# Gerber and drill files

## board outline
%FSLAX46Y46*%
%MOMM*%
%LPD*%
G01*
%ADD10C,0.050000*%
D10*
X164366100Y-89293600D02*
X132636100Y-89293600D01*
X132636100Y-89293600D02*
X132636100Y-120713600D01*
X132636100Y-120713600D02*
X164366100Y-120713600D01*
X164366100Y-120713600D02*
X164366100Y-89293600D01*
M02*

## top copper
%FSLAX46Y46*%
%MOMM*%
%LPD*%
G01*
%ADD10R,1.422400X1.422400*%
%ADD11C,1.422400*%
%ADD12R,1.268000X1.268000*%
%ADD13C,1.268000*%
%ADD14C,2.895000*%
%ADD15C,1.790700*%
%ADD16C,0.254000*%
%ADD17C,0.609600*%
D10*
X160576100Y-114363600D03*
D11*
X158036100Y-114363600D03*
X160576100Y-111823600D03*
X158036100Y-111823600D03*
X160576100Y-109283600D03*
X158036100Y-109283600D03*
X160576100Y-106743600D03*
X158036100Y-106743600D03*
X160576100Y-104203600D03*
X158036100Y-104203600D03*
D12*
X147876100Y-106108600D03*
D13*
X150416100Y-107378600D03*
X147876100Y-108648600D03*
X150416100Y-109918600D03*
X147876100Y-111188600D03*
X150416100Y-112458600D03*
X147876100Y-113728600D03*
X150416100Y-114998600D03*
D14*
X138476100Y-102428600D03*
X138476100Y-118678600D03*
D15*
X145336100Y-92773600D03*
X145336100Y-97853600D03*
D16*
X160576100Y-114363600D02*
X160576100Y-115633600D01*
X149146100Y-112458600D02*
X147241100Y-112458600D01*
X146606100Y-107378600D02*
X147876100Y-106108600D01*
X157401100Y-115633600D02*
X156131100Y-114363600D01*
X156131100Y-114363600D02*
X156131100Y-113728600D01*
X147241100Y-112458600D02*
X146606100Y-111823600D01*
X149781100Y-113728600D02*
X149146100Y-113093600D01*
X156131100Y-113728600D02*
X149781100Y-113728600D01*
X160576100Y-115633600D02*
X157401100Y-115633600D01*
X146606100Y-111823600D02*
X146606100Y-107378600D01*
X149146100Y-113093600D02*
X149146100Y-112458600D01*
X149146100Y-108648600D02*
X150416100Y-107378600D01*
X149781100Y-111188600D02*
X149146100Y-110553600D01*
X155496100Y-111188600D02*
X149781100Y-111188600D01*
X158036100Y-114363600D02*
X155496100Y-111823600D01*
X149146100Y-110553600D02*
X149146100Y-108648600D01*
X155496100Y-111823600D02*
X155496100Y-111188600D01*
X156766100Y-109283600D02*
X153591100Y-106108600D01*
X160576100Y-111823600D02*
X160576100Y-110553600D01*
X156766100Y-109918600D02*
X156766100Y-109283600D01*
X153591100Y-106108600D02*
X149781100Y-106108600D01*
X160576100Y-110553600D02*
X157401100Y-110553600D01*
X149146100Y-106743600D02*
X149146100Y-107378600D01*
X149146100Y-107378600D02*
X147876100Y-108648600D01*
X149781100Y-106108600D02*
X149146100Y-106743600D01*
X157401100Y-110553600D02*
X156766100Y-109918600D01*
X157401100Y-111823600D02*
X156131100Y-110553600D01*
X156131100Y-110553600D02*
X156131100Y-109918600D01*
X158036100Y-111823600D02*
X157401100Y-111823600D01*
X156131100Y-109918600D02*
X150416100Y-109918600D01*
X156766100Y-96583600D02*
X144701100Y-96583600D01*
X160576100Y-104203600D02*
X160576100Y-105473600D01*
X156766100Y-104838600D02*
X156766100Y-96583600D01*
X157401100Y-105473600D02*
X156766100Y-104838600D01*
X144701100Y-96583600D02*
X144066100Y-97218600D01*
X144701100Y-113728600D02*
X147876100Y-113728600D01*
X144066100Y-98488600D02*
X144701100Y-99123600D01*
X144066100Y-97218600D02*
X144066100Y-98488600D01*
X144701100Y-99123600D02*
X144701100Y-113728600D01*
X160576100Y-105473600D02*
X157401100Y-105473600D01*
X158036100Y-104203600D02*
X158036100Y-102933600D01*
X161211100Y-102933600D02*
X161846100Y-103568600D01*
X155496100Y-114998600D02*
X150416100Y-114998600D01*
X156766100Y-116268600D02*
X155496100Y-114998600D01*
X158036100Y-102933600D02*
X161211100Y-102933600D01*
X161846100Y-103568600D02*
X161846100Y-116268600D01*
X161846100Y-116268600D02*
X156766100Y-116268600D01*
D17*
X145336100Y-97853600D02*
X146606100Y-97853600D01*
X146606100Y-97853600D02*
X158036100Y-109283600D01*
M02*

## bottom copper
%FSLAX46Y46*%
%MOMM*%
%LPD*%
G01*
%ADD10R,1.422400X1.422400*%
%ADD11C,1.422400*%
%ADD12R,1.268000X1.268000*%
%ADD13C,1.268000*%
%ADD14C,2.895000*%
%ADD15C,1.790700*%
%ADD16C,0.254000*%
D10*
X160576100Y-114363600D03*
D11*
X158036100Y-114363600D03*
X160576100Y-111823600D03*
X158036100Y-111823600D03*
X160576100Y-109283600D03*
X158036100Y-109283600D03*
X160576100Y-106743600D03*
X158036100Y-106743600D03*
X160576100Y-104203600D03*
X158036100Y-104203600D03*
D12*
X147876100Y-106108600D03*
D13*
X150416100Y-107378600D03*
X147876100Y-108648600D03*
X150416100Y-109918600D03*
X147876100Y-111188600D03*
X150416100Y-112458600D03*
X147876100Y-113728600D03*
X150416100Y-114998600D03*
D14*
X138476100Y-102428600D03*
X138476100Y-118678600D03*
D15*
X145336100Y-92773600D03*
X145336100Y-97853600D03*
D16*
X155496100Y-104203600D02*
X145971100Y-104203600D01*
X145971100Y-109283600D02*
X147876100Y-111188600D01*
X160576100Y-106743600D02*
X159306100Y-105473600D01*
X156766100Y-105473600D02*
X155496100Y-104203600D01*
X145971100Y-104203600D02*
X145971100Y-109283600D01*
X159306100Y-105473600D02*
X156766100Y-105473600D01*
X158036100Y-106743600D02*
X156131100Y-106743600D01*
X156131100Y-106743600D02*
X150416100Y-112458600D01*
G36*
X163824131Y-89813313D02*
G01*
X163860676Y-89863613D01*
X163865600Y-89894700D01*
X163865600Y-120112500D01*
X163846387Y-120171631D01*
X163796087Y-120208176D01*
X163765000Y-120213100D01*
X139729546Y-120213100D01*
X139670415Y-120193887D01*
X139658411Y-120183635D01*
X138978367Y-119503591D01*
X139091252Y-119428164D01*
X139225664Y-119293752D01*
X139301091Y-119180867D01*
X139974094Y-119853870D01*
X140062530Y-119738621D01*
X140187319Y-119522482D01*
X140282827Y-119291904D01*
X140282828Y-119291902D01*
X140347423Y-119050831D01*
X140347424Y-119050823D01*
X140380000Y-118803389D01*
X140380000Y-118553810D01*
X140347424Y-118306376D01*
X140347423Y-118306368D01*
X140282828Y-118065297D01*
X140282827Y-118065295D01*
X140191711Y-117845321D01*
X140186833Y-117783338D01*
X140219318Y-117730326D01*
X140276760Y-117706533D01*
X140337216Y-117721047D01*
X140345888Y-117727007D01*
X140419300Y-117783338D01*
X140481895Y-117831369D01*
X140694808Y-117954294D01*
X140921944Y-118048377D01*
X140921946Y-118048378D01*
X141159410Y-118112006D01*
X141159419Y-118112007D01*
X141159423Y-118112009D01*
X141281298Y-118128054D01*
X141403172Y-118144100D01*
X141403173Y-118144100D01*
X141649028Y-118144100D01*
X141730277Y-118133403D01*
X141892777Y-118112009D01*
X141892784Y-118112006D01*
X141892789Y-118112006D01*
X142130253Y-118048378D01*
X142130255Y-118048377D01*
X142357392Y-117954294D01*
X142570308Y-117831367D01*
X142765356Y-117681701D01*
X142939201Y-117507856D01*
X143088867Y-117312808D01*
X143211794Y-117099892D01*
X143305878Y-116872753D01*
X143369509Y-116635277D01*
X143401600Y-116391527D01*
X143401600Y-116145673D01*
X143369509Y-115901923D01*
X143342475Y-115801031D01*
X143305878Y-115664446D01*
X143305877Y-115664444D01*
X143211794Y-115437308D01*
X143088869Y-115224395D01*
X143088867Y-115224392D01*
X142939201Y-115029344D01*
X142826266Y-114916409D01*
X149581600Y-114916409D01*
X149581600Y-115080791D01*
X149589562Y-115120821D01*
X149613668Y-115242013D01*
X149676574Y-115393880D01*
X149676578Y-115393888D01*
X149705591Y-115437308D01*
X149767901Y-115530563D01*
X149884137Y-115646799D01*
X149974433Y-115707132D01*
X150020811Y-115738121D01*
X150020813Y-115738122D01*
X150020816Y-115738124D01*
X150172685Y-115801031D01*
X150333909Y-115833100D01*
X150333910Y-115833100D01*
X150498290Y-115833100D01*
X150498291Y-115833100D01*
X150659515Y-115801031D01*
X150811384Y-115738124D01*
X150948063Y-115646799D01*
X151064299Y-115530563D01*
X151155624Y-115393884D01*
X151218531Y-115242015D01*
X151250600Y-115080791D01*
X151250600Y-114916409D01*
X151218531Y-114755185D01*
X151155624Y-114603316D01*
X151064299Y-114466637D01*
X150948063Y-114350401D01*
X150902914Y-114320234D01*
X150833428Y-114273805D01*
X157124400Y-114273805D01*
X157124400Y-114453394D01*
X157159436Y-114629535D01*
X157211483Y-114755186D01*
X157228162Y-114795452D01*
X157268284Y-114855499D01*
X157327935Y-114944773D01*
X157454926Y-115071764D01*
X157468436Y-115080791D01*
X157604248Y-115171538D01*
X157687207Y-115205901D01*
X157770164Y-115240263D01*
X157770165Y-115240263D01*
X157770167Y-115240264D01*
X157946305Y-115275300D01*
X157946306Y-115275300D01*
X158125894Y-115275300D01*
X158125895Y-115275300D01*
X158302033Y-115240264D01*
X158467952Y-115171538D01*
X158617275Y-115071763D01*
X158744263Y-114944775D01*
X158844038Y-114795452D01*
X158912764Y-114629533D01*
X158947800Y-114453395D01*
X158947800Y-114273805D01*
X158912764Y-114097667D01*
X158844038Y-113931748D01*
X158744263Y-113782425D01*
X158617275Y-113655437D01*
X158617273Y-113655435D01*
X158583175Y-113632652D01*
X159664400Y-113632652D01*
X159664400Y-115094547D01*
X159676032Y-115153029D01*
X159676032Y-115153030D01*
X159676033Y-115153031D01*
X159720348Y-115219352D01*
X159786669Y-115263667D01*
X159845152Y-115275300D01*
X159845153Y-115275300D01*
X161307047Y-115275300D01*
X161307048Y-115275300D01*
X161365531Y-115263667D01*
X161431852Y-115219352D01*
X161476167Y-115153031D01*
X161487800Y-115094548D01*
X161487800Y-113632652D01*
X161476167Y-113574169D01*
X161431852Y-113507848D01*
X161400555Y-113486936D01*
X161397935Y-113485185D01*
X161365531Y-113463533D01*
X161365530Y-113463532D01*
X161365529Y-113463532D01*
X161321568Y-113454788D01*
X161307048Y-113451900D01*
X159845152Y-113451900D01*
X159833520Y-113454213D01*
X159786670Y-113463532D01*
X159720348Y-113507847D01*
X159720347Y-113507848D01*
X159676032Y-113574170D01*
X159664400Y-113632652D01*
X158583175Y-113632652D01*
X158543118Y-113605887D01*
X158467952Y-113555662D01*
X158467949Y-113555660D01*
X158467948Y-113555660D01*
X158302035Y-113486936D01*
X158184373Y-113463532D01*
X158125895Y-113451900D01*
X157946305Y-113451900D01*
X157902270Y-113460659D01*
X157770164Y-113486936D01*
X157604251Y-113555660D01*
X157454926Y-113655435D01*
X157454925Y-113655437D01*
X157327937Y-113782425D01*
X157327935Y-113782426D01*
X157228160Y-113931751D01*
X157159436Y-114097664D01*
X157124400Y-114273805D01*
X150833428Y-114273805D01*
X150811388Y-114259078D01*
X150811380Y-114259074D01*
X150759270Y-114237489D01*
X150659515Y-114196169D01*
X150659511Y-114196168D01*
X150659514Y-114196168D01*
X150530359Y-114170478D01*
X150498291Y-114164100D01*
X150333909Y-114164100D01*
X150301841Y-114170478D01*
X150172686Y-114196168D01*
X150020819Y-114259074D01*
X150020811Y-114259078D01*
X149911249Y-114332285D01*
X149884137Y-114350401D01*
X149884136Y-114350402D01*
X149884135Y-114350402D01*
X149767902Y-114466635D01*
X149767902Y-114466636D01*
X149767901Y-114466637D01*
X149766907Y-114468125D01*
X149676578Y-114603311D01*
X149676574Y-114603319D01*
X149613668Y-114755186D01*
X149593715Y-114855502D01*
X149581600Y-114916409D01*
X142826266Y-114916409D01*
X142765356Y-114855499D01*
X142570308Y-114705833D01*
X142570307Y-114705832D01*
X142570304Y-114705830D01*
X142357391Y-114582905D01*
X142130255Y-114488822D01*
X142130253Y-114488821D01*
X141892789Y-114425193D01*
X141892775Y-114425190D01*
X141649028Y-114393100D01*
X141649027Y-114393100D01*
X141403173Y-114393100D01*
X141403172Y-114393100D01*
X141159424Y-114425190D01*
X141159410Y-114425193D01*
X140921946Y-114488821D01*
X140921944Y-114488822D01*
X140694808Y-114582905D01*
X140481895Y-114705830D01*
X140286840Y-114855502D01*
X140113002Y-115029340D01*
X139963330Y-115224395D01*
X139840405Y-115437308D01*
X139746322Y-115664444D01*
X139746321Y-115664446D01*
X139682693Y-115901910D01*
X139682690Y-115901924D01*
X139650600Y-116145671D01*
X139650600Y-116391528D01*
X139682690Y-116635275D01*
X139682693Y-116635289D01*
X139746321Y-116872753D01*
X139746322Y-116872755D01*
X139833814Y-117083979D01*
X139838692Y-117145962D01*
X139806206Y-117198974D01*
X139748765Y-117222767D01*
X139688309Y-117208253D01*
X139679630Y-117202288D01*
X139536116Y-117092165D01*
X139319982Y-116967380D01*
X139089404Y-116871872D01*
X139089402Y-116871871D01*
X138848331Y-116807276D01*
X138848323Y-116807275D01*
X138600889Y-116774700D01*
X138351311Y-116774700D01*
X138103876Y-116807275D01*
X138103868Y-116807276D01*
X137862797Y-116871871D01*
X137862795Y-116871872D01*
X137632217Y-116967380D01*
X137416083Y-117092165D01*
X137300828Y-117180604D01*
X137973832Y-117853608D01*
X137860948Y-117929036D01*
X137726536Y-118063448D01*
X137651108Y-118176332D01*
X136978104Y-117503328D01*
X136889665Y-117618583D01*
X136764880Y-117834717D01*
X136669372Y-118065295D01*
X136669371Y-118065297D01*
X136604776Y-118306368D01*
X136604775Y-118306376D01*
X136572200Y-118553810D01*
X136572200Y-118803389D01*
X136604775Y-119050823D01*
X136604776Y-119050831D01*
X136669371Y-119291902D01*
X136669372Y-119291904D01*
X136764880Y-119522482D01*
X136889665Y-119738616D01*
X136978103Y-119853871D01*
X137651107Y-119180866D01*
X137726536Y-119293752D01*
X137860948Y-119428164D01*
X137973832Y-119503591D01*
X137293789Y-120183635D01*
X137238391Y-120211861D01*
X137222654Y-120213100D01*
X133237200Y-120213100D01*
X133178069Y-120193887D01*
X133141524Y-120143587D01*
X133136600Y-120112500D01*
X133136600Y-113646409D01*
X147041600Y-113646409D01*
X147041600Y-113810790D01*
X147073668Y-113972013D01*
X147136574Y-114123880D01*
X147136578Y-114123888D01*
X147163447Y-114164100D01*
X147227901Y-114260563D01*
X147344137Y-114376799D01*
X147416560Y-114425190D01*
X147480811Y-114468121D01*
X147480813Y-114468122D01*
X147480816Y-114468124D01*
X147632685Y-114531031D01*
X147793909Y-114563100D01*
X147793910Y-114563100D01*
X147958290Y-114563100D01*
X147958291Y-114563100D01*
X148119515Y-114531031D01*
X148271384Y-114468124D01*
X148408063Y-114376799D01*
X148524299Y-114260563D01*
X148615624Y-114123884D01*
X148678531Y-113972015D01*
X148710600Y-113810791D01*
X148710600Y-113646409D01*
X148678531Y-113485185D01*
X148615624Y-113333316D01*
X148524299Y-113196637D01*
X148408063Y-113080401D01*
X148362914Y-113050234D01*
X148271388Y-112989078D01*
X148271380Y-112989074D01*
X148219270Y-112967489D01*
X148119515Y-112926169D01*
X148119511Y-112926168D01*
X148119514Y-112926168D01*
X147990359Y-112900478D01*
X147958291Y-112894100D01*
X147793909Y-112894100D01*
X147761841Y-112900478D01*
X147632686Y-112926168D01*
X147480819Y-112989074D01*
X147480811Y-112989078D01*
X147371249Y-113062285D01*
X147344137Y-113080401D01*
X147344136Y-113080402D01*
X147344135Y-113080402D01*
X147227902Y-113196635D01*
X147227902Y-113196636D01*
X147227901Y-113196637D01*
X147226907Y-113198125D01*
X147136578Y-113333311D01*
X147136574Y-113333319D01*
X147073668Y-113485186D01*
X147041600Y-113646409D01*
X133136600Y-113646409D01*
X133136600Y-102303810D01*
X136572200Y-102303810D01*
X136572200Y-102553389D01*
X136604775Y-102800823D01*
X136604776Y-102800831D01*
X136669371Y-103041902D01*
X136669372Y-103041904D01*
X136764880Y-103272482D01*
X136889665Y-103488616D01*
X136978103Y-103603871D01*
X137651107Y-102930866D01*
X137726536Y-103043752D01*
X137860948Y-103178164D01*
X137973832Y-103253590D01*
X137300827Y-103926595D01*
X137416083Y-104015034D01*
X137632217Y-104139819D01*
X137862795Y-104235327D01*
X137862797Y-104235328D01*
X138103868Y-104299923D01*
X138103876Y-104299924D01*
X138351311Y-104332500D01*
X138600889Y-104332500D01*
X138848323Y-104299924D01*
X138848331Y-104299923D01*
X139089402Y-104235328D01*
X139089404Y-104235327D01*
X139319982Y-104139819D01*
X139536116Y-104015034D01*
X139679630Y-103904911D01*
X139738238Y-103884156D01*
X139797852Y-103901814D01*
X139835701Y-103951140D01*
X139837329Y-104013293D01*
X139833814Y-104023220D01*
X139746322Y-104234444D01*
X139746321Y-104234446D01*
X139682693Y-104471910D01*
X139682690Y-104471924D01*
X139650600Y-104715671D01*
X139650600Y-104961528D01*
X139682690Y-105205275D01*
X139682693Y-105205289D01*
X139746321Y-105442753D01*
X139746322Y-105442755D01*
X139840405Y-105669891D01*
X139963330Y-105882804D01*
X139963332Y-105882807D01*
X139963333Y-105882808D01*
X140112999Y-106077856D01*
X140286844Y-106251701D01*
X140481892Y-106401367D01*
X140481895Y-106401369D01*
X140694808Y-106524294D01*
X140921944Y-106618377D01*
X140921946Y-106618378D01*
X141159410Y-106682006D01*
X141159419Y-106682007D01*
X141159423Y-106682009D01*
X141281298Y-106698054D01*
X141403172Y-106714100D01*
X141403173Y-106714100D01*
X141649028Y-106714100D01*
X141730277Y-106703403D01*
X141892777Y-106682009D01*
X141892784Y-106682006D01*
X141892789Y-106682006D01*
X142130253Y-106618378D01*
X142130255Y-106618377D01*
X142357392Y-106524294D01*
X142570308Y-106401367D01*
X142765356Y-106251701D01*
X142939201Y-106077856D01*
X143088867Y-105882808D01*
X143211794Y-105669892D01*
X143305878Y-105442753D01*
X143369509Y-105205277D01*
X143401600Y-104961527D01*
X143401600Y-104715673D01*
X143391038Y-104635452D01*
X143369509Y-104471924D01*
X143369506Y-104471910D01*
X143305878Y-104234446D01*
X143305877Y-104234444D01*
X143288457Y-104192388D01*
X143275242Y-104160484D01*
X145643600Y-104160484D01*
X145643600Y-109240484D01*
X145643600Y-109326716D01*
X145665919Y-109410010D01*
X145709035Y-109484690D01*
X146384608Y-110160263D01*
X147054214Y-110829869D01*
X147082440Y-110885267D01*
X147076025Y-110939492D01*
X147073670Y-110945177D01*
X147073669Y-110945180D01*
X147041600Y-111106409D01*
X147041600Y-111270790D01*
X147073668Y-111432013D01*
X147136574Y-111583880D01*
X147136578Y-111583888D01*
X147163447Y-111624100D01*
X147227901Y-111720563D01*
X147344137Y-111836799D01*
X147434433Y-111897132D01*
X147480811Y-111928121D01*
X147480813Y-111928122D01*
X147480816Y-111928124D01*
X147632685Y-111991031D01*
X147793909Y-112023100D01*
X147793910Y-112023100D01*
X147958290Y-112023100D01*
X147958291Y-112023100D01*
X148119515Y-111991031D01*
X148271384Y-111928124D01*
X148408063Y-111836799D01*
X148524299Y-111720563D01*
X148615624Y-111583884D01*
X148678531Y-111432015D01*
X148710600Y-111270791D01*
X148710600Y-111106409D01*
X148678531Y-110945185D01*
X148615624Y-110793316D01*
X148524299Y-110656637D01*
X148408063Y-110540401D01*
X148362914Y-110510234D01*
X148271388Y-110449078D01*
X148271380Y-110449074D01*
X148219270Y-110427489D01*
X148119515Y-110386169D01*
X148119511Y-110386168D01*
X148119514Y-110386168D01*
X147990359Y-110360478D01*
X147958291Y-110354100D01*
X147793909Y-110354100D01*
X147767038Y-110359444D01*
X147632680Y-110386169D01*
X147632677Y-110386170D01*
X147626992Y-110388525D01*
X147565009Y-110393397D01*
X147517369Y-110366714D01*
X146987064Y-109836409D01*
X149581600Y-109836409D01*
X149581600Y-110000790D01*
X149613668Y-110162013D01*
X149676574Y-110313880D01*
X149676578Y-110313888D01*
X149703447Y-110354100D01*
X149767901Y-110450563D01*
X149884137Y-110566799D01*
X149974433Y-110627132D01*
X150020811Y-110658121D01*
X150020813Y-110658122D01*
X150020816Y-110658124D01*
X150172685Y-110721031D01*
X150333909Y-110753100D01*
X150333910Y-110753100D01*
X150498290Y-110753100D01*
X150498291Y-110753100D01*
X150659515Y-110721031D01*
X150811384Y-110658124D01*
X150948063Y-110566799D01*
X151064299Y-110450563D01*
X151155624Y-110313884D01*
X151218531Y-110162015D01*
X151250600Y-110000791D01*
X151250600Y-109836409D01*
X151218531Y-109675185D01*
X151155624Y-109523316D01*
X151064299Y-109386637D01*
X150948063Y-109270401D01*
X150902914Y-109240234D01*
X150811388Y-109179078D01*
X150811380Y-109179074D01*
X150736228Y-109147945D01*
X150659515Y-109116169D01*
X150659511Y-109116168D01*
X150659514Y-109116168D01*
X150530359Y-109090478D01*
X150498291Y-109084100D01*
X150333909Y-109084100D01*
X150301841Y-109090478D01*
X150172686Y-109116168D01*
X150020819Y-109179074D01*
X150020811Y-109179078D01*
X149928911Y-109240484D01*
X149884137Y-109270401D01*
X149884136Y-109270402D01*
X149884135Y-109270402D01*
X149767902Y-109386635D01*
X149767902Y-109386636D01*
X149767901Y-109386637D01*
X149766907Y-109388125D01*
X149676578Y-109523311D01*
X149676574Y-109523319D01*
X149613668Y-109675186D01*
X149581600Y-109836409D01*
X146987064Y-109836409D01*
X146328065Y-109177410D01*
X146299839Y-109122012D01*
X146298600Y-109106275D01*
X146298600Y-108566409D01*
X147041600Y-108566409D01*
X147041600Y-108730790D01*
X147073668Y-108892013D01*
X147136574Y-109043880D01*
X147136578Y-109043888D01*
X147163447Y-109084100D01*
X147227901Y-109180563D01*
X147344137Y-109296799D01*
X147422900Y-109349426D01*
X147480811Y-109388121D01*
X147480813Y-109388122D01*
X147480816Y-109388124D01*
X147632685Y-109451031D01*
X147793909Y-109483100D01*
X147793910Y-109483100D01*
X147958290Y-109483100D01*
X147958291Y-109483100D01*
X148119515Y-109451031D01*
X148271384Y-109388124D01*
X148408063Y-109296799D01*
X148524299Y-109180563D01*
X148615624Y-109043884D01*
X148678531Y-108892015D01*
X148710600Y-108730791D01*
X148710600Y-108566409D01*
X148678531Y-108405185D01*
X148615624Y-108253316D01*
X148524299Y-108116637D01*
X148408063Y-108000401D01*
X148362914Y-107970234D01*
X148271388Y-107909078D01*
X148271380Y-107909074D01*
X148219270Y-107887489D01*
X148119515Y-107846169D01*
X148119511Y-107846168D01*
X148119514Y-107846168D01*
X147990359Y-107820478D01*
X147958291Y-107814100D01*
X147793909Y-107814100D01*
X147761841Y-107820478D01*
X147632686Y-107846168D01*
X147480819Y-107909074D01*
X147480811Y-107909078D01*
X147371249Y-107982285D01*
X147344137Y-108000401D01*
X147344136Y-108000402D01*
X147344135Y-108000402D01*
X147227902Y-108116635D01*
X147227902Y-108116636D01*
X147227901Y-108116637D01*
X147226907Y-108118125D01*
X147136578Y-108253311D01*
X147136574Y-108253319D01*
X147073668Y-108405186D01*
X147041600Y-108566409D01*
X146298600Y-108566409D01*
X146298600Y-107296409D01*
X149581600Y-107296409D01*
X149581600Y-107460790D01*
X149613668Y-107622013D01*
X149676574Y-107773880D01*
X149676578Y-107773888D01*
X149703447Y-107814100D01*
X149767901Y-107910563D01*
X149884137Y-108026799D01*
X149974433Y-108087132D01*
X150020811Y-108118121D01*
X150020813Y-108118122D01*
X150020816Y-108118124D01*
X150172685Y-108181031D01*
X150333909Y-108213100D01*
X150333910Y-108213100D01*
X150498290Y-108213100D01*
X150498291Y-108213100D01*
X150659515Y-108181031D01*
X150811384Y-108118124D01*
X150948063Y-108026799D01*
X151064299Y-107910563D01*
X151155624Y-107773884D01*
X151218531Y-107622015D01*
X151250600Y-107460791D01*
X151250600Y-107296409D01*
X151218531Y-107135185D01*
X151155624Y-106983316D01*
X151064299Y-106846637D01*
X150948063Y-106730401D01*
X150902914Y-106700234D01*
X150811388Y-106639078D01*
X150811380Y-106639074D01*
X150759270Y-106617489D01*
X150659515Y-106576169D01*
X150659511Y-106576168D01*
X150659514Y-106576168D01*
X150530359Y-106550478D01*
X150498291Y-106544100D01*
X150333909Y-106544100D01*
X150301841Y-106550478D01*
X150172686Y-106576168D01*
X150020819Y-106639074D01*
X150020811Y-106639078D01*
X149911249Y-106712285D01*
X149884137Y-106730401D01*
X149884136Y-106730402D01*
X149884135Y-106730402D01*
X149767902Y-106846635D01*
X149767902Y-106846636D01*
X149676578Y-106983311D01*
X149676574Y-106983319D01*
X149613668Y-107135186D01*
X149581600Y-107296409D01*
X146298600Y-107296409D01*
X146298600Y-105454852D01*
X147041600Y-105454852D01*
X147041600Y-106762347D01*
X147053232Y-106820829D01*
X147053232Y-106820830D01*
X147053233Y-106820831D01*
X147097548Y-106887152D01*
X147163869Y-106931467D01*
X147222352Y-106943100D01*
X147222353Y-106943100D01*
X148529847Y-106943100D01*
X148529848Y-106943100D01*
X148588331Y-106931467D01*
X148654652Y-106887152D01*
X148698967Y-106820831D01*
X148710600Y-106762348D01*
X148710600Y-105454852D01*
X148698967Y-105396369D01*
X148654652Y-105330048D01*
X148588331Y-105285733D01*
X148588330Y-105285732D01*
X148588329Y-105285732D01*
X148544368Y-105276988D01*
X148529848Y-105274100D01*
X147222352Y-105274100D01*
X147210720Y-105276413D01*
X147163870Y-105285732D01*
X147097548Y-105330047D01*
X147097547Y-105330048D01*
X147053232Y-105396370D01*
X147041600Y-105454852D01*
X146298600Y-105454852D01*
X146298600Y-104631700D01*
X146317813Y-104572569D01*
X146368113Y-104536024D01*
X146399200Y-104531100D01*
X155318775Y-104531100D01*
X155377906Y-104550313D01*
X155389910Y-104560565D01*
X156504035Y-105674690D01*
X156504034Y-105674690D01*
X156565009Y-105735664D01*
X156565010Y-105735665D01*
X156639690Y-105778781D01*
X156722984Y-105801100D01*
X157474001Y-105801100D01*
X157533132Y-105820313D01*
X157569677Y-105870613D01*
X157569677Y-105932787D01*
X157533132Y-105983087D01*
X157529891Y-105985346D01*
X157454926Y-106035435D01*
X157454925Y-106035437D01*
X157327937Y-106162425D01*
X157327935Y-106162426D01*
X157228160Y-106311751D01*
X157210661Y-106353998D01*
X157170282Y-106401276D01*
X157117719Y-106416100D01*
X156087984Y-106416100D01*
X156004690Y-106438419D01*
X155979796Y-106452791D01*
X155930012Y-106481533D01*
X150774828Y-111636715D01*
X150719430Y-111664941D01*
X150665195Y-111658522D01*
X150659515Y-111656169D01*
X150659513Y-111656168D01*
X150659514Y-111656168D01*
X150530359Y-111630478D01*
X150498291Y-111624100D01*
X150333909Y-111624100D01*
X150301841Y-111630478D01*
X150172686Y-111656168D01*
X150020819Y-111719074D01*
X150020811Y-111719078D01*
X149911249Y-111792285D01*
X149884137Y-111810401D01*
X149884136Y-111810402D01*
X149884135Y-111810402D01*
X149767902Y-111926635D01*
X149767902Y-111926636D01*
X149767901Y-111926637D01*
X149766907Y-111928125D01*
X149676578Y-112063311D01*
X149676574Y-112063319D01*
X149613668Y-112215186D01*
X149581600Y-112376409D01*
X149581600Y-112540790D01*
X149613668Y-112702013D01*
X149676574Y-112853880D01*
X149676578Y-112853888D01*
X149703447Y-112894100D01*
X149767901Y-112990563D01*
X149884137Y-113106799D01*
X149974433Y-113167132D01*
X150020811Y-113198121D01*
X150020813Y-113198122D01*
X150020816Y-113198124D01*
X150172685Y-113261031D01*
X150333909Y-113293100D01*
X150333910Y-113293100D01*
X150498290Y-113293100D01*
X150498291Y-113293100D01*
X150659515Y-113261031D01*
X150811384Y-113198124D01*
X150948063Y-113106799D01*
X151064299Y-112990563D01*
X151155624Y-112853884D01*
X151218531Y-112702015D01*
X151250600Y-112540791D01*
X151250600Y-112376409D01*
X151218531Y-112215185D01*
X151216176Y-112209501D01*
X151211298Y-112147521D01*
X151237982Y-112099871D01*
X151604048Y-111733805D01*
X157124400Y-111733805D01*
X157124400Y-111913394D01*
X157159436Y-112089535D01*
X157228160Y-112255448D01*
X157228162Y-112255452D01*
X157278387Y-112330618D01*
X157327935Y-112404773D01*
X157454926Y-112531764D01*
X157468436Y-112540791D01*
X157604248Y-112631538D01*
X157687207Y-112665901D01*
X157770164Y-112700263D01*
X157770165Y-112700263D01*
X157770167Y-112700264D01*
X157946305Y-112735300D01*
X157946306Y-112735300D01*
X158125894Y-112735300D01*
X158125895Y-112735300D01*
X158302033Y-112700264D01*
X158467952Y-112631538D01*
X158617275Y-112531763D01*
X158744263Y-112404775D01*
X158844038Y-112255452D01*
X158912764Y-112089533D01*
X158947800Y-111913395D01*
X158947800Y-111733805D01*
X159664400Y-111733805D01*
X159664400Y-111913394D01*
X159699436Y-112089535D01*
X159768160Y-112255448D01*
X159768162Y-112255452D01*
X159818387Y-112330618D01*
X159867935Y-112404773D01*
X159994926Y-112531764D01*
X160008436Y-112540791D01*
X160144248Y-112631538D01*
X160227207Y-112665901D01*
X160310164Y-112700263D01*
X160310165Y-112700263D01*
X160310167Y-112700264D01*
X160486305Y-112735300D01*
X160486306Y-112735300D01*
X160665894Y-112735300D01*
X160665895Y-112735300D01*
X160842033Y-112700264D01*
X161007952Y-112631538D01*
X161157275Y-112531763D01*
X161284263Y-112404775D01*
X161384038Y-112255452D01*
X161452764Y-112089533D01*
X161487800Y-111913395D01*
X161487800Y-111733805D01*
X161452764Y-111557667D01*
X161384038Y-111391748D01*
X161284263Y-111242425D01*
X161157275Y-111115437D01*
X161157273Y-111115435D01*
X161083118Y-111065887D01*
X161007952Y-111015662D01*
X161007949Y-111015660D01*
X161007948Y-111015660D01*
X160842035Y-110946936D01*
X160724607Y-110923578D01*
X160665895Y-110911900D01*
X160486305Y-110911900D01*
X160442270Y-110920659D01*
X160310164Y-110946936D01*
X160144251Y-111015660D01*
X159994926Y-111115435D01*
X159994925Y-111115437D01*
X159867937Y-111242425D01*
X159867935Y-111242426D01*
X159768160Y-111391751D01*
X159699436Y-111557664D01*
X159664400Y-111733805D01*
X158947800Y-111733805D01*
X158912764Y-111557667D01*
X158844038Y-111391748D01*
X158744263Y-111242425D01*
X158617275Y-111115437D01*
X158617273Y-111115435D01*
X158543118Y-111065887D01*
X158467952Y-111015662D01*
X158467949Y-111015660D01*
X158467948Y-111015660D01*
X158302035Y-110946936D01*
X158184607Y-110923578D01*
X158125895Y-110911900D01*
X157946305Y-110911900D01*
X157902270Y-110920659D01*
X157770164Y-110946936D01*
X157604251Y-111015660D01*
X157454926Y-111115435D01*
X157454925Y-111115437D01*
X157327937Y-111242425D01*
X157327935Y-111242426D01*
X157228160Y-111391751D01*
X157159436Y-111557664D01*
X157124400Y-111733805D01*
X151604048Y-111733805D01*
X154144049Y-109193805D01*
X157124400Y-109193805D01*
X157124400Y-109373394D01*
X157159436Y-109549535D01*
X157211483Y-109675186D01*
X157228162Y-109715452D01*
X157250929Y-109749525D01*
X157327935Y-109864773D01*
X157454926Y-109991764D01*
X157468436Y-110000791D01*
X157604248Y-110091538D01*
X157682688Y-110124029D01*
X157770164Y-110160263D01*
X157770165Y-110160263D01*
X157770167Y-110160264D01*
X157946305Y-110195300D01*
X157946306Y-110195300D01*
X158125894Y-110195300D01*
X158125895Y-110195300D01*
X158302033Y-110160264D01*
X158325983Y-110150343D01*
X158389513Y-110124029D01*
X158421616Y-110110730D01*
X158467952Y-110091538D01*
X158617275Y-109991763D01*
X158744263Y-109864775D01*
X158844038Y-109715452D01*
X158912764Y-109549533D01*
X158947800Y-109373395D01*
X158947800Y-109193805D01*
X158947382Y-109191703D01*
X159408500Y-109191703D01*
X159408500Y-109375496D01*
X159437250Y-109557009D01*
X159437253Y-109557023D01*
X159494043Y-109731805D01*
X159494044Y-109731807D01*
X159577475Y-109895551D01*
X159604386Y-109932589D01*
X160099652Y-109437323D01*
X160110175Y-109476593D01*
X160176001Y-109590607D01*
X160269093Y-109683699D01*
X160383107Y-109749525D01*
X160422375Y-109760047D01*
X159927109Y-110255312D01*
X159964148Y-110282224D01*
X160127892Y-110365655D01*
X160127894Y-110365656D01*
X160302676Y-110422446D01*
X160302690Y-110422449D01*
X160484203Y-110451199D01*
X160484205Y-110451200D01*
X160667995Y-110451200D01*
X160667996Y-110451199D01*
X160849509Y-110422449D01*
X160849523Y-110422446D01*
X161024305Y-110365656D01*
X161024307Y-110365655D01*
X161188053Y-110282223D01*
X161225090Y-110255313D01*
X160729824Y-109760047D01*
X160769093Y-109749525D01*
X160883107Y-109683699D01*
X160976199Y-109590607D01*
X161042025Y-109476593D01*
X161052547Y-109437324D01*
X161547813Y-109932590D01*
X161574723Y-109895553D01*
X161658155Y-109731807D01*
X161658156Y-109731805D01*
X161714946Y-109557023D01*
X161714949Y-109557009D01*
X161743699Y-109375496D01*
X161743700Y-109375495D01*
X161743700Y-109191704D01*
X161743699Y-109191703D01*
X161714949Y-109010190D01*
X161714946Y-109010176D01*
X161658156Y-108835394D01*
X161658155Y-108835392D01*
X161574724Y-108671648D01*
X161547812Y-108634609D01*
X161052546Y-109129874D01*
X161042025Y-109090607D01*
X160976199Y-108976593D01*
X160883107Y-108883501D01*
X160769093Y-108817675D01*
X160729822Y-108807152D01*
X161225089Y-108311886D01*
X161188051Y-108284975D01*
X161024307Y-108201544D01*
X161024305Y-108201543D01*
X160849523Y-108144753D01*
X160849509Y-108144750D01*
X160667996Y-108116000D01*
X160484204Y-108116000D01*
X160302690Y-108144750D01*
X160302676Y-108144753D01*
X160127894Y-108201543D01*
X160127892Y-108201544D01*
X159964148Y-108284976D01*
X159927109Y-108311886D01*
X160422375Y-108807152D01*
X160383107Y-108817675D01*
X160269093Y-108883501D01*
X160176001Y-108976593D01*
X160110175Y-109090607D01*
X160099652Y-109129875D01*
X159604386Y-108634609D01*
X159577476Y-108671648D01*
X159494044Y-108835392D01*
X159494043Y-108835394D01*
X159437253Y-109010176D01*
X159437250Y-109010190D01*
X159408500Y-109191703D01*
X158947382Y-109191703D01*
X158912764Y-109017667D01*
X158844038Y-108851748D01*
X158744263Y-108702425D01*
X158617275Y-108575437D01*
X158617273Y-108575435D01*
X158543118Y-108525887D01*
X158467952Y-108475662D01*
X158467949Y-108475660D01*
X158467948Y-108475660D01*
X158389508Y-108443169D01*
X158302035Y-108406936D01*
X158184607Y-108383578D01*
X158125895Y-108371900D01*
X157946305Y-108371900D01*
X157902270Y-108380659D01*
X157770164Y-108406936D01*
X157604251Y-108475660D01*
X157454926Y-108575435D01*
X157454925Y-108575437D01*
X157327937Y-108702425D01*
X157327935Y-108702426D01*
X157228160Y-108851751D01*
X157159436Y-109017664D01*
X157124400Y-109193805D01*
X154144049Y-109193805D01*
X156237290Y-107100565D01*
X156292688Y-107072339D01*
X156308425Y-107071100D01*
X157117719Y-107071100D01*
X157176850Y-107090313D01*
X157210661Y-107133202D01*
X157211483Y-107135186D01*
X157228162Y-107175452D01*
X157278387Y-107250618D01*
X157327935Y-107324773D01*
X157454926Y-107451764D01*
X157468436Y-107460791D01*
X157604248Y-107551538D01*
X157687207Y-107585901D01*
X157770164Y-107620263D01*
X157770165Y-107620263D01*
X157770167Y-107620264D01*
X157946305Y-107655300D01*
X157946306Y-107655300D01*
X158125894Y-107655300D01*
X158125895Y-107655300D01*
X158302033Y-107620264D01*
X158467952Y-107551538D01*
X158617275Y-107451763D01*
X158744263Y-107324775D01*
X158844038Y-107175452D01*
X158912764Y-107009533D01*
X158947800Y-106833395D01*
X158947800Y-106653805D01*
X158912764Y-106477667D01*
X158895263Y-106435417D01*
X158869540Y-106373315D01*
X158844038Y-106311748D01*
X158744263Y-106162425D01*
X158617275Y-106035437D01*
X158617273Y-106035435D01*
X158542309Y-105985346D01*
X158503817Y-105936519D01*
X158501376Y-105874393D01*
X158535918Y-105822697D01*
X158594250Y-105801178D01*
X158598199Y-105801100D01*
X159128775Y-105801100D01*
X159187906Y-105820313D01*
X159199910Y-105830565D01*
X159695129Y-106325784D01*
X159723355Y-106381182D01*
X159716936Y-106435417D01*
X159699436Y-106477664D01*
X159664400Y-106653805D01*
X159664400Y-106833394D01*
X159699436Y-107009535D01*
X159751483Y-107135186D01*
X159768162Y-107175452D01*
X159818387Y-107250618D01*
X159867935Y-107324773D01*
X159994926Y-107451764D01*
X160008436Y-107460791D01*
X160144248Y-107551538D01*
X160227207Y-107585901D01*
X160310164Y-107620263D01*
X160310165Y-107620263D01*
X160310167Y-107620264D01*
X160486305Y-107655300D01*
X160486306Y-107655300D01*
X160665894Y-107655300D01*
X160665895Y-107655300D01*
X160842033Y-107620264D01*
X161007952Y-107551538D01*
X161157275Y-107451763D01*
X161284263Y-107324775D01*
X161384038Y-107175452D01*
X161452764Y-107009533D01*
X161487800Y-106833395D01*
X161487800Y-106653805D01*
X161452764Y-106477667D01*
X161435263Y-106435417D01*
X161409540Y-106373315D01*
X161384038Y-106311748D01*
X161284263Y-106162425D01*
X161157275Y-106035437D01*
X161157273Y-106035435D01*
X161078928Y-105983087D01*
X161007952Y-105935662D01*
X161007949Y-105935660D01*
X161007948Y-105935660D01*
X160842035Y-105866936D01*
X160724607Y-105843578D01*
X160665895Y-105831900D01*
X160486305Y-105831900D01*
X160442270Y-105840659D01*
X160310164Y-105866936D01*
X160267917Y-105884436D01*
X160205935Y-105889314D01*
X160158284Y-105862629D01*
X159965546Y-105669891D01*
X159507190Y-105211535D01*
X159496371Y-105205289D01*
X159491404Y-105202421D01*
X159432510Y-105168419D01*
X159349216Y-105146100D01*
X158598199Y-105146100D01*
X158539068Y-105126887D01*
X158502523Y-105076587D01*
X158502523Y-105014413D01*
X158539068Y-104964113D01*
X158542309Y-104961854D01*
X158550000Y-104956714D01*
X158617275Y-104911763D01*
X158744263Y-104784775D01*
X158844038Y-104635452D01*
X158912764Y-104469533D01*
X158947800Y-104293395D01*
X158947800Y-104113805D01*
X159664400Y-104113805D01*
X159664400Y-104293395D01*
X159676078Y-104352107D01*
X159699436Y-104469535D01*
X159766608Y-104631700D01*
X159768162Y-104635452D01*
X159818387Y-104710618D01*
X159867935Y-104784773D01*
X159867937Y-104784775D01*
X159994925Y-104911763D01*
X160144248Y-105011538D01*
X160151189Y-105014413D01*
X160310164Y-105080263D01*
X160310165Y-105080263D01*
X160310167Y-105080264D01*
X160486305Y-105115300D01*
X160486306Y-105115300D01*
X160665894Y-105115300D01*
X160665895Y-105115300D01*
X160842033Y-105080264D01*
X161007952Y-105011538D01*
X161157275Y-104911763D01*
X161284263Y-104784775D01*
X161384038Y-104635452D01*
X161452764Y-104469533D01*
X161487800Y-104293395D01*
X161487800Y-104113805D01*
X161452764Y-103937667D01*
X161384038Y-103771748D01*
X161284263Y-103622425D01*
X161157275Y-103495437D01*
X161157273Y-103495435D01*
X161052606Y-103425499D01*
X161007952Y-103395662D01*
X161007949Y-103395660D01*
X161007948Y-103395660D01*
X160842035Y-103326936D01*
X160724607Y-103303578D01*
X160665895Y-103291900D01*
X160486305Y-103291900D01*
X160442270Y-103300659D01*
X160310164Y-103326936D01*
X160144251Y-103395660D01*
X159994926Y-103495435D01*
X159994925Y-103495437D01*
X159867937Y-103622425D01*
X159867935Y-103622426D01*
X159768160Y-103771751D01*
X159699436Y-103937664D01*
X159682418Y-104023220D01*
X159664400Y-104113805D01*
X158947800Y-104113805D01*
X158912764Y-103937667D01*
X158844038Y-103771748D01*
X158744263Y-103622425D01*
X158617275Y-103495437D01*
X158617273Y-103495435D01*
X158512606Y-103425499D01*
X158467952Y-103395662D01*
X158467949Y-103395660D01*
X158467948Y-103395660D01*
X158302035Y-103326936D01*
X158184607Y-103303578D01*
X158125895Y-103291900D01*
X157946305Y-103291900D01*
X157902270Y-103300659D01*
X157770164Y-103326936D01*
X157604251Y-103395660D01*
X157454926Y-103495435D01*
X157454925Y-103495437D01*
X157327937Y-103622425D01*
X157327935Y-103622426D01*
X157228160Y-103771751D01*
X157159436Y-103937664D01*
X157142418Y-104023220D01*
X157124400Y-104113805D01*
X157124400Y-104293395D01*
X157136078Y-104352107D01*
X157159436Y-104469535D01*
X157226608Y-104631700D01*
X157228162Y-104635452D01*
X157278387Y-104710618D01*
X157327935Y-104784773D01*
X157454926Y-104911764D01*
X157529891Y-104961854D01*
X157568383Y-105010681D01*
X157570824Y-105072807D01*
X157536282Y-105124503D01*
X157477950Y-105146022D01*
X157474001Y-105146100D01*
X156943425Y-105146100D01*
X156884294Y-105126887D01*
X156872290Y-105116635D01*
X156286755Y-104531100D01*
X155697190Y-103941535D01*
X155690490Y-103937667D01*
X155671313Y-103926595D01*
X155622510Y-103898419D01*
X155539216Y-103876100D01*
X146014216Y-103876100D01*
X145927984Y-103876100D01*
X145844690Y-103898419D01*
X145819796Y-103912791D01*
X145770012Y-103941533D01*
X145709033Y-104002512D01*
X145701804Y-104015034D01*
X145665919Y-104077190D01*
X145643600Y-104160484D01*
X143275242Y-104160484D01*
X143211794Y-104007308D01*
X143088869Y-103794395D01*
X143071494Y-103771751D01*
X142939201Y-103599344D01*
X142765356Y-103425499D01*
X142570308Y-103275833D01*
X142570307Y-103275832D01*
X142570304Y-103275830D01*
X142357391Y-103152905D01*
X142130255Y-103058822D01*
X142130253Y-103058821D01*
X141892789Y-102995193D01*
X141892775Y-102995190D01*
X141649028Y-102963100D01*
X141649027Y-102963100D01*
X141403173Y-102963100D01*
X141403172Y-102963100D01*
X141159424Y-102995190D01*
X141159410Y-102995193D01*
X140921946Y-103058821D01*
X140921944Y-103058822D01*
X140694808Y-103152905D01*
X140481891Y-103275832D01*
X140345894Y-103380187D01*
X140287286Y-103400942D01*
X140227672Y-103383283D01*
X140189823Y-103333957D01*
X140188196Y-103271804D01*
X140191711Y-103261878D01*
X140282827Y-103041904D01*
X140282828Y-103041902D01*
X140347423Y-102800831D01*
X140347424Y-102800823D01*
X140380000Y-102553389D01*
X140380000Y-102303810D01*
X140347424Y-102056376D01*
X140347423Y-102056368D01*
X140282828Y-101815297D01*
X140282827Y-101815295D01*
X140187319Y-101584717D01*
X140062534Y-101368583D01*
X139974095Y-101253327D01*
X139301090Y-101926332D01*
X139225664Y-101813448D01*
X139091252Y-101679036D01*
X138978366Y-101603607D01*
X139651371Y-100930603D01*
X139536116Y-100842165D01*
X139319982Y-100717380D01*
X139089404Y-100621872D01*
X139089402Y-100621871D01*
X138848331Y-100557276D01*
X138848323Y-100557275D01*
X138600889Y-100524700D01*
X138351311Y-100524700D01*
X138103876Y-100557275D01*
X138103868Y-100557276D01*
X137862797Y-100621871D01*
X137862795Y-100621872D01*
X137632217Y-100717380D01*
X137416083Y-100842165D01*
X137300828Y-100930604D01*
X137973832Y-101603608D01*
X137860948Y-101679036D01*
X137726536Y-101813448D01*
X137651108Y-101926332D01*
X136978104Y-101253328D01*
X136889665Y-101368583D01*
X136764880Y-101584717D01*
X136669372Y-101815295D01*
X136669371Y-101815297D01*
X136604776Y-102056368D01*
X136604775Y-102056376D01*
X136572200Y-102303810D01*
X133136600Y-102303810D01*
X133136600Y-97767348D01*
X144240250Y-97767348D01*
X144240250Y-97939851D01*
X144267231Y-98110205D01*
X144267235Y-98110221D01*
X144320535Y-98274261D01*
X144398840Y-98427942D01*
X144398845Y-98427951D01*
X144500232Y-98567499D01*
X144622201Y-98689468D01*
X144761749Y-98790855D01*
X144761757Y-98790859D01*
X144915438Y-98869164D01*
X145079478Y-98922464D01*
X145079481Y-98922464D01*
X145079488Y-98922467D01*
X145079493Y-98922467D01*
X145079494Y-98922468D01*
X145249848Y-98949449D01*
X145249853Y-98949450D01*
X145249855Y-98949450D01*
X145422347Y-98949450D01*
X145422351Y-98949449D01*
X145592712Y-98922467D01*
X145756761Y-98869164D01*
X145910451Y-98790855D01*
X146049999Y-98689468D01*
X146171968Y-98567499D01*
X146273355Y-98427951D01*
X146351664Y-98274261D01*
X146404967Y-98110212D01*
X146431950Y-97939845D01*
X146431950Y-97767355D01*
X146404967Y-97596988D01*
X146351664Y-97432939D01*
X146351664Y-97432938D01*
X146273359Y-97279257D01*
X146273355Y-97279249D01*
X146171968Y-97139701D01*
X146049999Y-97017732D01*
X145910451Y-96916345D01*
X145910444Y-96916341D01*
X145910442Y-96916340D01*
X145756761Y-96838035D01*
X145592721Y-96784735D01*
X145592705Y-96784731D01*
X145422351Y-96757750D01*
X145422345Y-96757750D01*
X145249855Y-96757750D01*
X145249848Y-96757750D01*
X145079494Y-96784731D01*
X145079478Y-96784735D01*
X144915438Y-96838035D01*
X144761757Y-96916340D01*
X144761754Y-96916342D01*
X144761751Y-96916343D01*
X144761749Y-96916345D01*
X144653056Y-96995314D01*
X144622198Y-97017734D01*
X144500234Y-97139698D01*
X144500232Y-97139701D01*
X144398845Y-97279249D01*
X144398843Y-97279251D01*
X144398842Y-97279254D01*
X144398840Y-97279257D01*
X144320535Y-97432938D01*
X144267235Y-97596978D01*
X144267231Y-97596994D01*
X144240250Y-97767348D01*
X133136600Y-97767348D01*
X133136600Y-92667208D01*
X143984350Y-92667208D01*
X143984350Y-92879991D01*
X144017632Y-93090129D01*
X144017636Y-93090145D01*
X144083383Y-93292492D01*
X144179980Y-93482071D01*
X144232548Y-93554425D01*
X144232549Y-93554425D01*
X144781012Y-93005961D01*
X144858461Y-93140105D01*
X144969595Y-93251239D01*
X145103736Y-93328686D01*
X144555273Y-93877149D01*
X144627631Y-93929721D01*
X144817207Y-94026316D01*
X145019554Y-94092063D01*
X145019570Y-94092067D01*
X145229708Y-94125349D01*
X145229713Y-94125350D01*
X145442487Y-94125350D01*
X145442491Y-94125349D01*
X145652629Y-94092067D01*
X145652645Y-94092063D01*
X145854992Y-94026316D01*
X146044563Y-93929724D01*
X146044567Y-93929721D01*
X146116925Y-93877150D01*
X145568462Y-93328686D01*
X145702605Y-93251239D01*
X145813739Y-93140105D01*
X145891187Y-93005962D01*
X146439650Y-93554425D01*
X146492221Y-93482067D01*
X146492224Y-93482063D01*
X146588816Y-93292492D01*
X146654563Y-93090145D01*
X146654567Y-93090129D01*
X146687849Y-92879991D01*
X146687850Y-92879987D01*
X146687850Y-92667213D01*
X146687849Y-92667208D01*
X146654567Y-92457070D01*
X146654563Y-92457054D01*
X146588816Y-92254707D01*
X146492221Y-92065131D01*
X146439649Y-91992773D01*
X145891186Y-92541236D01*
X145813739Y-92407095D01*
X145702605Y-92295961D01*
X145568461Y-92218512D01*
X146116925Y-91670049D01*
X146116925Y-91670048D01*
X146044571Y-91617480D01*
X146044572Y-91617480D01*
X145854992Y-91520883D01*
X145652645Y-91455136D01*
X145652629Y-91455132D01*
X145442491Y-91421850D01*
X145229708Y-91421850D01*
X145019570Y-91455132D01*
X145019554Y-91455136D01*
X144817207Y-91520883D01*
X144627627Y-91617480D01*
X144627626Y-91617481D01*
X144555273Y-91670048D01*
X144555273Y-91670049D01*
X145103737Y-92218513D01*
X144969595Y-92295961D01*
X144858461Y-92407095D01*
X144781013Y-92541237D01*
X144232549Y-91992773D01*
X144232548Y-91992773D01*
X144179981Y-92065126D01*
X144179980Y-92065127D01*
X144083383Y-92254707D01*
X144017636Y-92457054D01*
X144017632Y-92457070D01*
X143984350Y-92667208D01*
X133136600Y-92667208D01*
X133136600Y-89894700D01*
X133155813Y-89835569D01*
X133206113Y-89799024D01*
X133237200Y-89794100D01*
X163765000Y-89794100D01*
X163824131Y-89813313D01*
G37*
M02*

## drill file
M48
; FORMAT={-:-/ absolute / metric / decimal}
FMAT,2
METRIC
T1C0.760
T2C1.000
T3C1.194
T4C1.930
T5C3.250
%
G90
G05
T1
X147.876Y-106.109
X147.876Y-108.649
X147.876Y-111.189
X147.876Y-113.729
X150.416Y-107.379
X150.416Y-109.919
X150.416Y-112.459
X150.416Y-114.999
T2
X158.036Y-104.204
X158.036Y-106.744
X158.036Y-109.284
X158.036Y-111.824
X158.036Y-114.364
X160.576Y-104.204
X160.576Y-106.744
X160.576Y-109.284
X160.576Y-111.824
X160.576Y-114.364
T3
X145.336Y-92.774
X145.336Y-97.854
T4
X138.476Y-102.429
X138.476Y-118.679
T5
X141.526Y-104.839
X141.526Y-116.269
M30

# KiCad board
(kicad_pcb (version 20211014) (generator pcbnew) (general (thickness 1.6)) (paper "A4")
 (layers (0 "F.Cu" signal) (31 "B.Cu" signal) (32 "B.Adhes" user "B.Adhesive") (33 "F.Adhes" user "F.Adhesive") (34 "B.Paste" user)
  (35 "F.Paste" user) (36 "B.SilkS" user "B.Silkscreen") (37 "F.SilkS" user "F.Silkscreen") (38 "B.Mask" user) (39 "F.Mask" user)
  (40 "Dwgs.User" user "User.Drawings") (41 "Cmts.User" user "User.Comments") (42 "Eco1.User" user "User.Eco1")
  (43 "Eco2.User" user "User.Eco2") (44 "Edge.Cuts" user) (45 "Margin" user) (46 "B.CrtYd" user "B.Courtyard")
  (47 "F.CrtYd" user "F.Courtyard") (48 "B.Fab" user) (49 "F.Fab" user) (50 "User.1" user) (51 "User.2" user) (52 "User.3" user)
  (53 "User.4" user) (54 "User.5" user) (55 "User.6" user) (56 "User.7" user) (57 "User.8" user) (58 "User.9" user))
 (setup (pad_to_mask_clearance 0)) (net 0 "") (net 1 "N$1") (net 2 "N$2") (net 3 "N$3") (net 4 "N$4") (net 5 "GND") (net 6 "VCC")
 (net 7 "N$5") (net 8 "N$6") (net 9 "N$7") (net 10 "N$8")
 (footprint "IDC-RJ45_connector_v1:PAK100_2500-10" (layer "F.Cu") (at 159.3061 109.2836 90)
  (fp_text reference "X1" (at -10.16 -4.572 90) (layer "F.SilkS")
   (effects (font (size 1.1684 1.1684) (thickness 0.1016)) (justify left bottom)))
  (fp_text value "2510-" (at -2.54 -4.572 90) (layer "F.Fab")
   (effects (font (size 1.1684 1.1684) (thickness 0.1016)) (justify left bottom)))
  (pad "1" thru_hole rect (at -5.08 1.27 90) (size 1.4224 1.4224) (drill 1) (layers *.Cu *.Mask) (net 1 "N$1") (solder_mask_margin 0.1016))
  (pad "2" thru_hole circle (at -5.08 -1.27 90) (size 1.4224 1.4224) (drill 1) (layers *.Cu *.Mask) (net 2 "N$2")
   (solder_mask_margin 0.1016))
  (pad "3" thru_hole circle (at -2.54 1.27 90) (size 1.4224 1.4224) (drill 1) (layers *.Cu *.Mask) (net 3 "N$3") (solder_mask_margin 0.1016))
  (pad "4" thru_hole circle (at -2.54 -1.27 90) (size 1.4224 1.4224) (drill 1) (layers *.Cu *.Mask) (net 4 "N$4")
   (solder_mask_margin 0.1016))
  (pad "5" thru_hole circle (at 0 1.27 90) (size 1.4224 1.4224) (drill 1) (layers *.Cu *.Mask) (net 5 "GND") (solder_mask_margin 0.1016))
  (pad "6" thru_hole circle (at 0 -1.27 90) (size 1.4224 1.4224) (drill 1) (layers *.Cu *.Mask) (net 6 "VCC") (solder_mask_margin 0.1016))
  (pad "7" thru_hole circle (at 2.54 1.27 90) (size 1.4224 1.4224) (drill 1) (layers *.Cu *.Mask) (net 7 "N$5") (solder_mask_margin 0.1016))
  (pad "8" thru_hole circle (at 2.54 -1.27 90) (size 1.4224 1.4224) (drill 1) (layers *.Cu *.Mask) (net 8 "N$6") (solder_mask_margin 0.1016))
  (pad "9" thru_hole circle (at 5.08 1.27 90) (size 1.4224 1.4224) (drill 1) (layers *.Cu *.Mask) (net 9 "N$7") (solder_mask_margin 0.1016))
  (pad "10" thru_hole circle (at 5.08 -1.27 90) (size 1.4224 1.4224) (drill 1) (layers *.Cu *.Mask) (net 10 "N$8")
   (solder_mask_margin 0.1016)))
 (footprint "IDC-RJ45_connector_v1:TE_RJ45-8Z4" (layer "F.Cu") (at 141.5261 110.5536 -90)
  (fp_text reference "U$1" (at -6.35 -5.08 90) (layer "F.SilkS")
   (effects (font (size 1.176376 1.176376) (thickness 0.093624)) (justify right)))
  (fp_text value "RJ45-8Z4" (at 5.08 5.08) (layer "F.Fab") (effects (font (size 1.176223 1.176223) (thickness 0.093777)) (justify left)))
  (pad "" np_thru_hole circle (at 5.715 0 270) (size 3.25 3.25) (drill 3.25) (layers *.Cu *.Mask))
  (pad "" np_thru_hole circle (at -5.715 0 270) (size 3.25 3.25) (drill 3.25) (layers *.Cu *.Mask))
  (pad "1" thru_hole rect (at -4.445 -6.35 270) (size 1.268 1.268) (drill 0.76) (layers *.Cu *.Mask) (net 1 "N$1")
   (solder_mask_margin 0.1016))
  (pad "2" thru_hole circle (at -3.175 -8.89 270) (size 1.268 1.268) (drill 0.76) (layers *.Cu *.Mask) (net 2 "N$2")
   (solder_mask_margin 0.1016))
  (pad "3" thru_hole circle (at -1.905 -6.35 270) (size 1.268 1.268) (drill 0.76) (layers *.Cu *.Mask) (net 3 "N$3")
   (solder_mask_margin 0.1016))
  (pad "4" thru_hole circle (at -0.635 -8.89 270) (size 1.268 1.268) (drill 0.76) (layers *.Cu *.Mask) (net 4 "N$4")
   (solder_mask_margin 0.1016))
  (pad "5" thru_hole circle (at 0.635 -6.35 270) (size 1.268 1.268) (drill 0.76) (layers *.Cu *.Mask) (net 7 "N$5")
   (solder_mask_margin 0.1016))
  (pad "6" thru_hole circle (at 1.905 -8.89 270) (size 1.268 1.268) (drill 0.76) (layers *.Cu *.Mask) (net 8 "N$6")
   (solder_mask_margin 0.1016))
  (pad "7" thru_hole circle (at 3.175 -6.35 270) (size 1.268 1.268) (drill 0.76) (layers *.Cu *.Mask) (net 9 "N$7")
   (solder_mask_margin 0.1016))
  (pad "8" thru_hole circle (at 4.445 -8.89 270) (size 1.268 1.268) (drill 0.76) (layers *.Cu *.Mask) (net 10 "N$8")
   (solder_mask_margin 0.1016))
  (pad "9" thru_hole circle (at -8.125 3.05) (size 2.895 2.895) (drill 1.93) (layers *.Cu *.Mask) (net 5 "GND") (solder_mask_margin 0.1016))
  (pad "10" thru_hole circle (at 8.125 3.05) (size 2.895 2.895) (drill 1.93) (layers *.Cu *.Mask) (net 5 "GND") (solder_mask_margin 0.1016)))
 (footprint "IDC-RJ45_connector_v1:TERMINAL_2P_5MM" (layer "F.Cu") (at 145.3361 95.3136 -90)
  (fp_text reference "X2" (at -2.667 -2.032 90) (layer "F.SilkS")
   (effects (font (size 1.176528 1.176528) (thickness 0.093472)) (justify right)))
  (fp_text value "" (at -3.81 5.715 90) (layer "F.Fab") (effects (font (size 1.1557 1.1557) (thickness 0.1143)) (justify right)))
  (pad "1" thru_hole circle (at -2.54 0) (size 1.7907 1.7907) (drill 1.1938) (layers *.Cu *.Mask) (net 5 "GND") (solder_mask_margin 0.1016))
  (pad "2" thru_hole circle (at 2.54 0) (size 1.7907 1.7907) (drill 1.1938) (layers *.Cu *.Mask) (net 6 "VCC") (solder_mask_margin 0.1016)))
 (gr_line (start 164.3661 89.2936) (end 132.6361 89.2936) (layer "Edge.Cuts") (width 0.05))
 (gr_line (start 132.6361 89.2936) (end 132.6361 120.7136) (layer "Edge.Cuts") (width 0.05))
 (gr_line (start 132.6361 120.7136) (end 164.3661 120.7136) (layer "Edge.Cuts") (width 0.05))
 (gr_line (start 164.3661 120.7136) (end 164.3661 89.2936) (layer "Edge.Cuts") (width 0.05))
 (segment (start 160.5761 114.3636) (end 160.5761 115.6336) (width 0.254) (layer "F.Cu") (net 1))
 (segment (start 149.1461 112.4586) (end 147.2411 112.4586) (width 0.254) (layer "F.Cu") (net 1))
 (segment (start 146.6061 107.3786) (end 147.8761 106.1086) (width 0.254) (layer "F.Cu") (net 1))
 (segment (start 157.4011 115.6336) (end 156.1311 114.3636) (width 0.254) (layer "F.Cu") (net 1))
 (segment (start 156.1311 114.3636) (end 156.1311 113.7286) (width 0.254) (layer "F.Cu") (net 1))
 (segment (start 147.2411 112.4586) (end 146.6061 111.8236) (width 0.254) (layer "F.Cu") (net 1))
 (segment (start 149.7811 113.7286) (end 149.1461 113.0936) (width 0.254) (layer "F.Cu") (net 1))
 (segment (start 156.1311 113.7286) (end 149.7811 113.7286) (width 0.254) (layer "F.Cu") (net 1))
 (segment (start 160.5761 115.6336) (end 157.4011 115.6336) (width 0.254) (layer "F.Cu") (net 1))
 (segment (start 146.6061 111.8236) (end 146.6061 107.3786) (width 0.254) (layer "F.Cu") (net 1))
 (segment (start 149.1461 113.0936) (end 149.1461 112.4586) (width 0.254) (layer "F.Cu") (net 1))
 (segment (start 149.1461 108.6486) (end 150.4161 107.3786) (width 0.254) (layer "F.Cu") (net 2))
 (segment (start 149.7811 111.1886) (end 149.1461 110.5536) (width 0.254) (layer "F.Cu") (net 2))
 (segment (start 155.4961 111.1886) (end 149.7811 111.1886) (width 0.254) (layer "F.Cu") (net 2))
 (segment (start 158.0361 114.3636) (end 155.4961 111.8236) (width 0.254) (layer "F.Cu") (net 2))
 (segment (start 149.1461 110.5536) (end 149.1461 108.6486) (width 0.254) (layer "F.Cu") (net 2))
 (segment (start 155.4961 111.8236) (end 155.4961 111.1886) (width 0.254) (layer "F.Cu") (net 2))
 (segment (start 156.7661 109.2836) (end 153.5911 106.1086) (width 0.254) (layer "F.Cu") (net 3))
 (segment (start 160.5761 111.8236) (end 160.5761 110.5536) (width 0.254) (layer "F.Cu") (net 3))
 (segment (start 156.7661 109.9186) (end 156.7661 109.2836) (width 0.254) (layer "F.Cu") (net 3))
 (segment (start 153.5911 106.1086) (end 149.7811 106.1086) (width 0.254) (layer "F.Cu") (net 3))
 (segment (start 160.5761 110.5536) (end 157.4011 110.5536) (width 0.254) (layer "F.Cu") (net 3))
 (segment (start 149.1461 106.7436) (end 149.1461 107.3786) (width 0.254) (layer "F.Cu") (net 3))
 (segment (start 149.1461 107.3786) (end 147.8761 108.6486) (width 0.254) (layer "F.Cu") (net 3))
 (segment (start 149.7811 106.1086) (end 149.1461 106.7436) (width 0.254) (layer "F.Cu") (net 3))
 (segment (start 157.4011 110.5536) (end 156.7661 109.9186) (width 0.254) (layer "F.Cu") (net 3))
 (segment (start 157.4011 111.8236) (end 156.1311 110.5536) (width 0.254) (layer "F.Cu") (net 4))
 (segment (start 156.1311 110.5536) (end 156.1311 109.9186) (width 0.254) (layer "F.Cu") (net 4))
 (segment (start 158.0361 111.8236) (end 157.4011 111.8236) (width 0.254) (layer "F.Cu") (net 4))
 (segment (start 156.1311 109.9186) (end 150.4161 109.9186) (width 0.254) (layer "F.Cu") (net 4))
 (segment (start 155.4961 104.2036) (end 145.9711 104.2036) (width 0.254) (layer "B.Cu") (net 7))
 (segment (start 145.9711 109.2836) (end 147.8761 111.1886) (width 0.254) (layer "B.Cu") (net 7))
 (segment (start 160.5761 106.7436) (end 159.3061 105.4736) (width 0.254) (layer "B.Cu") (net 7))
 (segment (start 156.7661 105.4736) (end 155.4961 104.2036) (width 0.254) (layer "B.Cu") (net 7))
 (segment (start 145.9711 104.2036) (end 145.9711 109.2836) (width 0.254) (layer "B.Cu") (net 7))
 (segment (start 159.3061 105.4736) (end 156.7661 105.4736) (width 0.254) (layer "B.Cu") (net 7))
 (segment (start 158.0361 106.7436) (end 156.1311 106.7436) (width 0.254) (layer "B.Cu") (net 8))
 (segment (start 156.1311 106.7436) (end 150.4161 112.4586) (width 0.254) (layer "B.Cu") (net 8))
 (segment (start 156.7661 96.5836) (end 144.7011 96.5836) (width 0.254) (layer "F.Cu") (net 9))
 (segment (start 160.5761 104.2036) (end 160.5761 105.4736) (width 0.254) (layer "F.Cu") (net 9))
 (segment (start 156.7661 104.8386) (end 156.7661 96.5836) (width 0.254) (layer "F.Cu") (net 9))
 (segment (start 157.4011 105.4736) (end 156.7661 104.8386) (width 0.254) (layer "F.Cu") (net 9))
 (segment (start 144.7011 96.5836) (end 144.0661 97.2186) (width 0.254) (layer "F.Cu") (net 9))
 (segment (start 144.7011 113.7286) (end 147.8761 113.7286) (width 0.254) (layer "F.Cu") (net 9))
 (segment (start 144.0661 98.4886) (end 144.7011 99.1236) (width 0.254) (layer "F.Cu") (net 9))
 (segment (start 144.0661 97.2186) (end 144.0661 98.4886) (width 0.254) (layer "F.Cu") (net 9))
 (segment (start 144.7011 99.1236) (end 144.7011 113.7286) (width 0.254) (layer "F.Cu") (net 9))
 (segment (start 160.5761 105.4736) (end 157.4011 105.4736) (width 0.254) (layer "F.Cu") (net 9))
 (segment (start 158.0361 104.2036) (end 158.0361 102.9336) (width 0.254) (layer "F.Cu") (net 10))
 (segment (start 161.2111 102.9336) (end 161.8461 103.5686) (width 0.254) (layer "F.Cu") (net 10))
 (segment (start 155.4961 114.9986) (end 150.4161 114.9986) (width 0.254) (layer "F.Cu") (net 10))
 (segment (start 156.7661 116.2686) (end 155.4961 114.9986) (width 0.254) (layer "F.Cu") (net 10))
 (segment (start 158.0361 102.9336) (end 161.2111 102.9336) (width 0.254) (layer "F.Cu") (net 10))
 (segment (start 161.8461 103.5686) (end 161.8461 116.2686) (width 0.254) (layer "F.Cu") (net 10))
 (segment (start 161.8461 116.2686) (end 156.7661 116.2686) (width 0.254) (layer "F.Cu") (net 10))
 (segment (start 145.3361 97.8536) (end 146.6061 97.8536) (width 0.6096) (layer "F.Cu") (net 6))
 (segment (start 146.6061 97.8536) (end 158.0361 109.2836) (width 0.6096) (layer "F.Cu") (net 6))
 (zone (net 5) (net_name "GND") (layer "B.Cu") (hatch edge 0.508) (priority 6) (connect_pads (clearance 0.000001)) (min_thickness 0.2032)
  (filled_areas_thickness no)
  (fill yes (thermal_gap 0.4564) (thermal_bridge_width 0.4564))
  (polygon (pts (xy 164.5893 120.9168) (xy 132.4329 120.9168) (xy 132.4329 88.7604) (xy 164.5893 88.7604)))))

